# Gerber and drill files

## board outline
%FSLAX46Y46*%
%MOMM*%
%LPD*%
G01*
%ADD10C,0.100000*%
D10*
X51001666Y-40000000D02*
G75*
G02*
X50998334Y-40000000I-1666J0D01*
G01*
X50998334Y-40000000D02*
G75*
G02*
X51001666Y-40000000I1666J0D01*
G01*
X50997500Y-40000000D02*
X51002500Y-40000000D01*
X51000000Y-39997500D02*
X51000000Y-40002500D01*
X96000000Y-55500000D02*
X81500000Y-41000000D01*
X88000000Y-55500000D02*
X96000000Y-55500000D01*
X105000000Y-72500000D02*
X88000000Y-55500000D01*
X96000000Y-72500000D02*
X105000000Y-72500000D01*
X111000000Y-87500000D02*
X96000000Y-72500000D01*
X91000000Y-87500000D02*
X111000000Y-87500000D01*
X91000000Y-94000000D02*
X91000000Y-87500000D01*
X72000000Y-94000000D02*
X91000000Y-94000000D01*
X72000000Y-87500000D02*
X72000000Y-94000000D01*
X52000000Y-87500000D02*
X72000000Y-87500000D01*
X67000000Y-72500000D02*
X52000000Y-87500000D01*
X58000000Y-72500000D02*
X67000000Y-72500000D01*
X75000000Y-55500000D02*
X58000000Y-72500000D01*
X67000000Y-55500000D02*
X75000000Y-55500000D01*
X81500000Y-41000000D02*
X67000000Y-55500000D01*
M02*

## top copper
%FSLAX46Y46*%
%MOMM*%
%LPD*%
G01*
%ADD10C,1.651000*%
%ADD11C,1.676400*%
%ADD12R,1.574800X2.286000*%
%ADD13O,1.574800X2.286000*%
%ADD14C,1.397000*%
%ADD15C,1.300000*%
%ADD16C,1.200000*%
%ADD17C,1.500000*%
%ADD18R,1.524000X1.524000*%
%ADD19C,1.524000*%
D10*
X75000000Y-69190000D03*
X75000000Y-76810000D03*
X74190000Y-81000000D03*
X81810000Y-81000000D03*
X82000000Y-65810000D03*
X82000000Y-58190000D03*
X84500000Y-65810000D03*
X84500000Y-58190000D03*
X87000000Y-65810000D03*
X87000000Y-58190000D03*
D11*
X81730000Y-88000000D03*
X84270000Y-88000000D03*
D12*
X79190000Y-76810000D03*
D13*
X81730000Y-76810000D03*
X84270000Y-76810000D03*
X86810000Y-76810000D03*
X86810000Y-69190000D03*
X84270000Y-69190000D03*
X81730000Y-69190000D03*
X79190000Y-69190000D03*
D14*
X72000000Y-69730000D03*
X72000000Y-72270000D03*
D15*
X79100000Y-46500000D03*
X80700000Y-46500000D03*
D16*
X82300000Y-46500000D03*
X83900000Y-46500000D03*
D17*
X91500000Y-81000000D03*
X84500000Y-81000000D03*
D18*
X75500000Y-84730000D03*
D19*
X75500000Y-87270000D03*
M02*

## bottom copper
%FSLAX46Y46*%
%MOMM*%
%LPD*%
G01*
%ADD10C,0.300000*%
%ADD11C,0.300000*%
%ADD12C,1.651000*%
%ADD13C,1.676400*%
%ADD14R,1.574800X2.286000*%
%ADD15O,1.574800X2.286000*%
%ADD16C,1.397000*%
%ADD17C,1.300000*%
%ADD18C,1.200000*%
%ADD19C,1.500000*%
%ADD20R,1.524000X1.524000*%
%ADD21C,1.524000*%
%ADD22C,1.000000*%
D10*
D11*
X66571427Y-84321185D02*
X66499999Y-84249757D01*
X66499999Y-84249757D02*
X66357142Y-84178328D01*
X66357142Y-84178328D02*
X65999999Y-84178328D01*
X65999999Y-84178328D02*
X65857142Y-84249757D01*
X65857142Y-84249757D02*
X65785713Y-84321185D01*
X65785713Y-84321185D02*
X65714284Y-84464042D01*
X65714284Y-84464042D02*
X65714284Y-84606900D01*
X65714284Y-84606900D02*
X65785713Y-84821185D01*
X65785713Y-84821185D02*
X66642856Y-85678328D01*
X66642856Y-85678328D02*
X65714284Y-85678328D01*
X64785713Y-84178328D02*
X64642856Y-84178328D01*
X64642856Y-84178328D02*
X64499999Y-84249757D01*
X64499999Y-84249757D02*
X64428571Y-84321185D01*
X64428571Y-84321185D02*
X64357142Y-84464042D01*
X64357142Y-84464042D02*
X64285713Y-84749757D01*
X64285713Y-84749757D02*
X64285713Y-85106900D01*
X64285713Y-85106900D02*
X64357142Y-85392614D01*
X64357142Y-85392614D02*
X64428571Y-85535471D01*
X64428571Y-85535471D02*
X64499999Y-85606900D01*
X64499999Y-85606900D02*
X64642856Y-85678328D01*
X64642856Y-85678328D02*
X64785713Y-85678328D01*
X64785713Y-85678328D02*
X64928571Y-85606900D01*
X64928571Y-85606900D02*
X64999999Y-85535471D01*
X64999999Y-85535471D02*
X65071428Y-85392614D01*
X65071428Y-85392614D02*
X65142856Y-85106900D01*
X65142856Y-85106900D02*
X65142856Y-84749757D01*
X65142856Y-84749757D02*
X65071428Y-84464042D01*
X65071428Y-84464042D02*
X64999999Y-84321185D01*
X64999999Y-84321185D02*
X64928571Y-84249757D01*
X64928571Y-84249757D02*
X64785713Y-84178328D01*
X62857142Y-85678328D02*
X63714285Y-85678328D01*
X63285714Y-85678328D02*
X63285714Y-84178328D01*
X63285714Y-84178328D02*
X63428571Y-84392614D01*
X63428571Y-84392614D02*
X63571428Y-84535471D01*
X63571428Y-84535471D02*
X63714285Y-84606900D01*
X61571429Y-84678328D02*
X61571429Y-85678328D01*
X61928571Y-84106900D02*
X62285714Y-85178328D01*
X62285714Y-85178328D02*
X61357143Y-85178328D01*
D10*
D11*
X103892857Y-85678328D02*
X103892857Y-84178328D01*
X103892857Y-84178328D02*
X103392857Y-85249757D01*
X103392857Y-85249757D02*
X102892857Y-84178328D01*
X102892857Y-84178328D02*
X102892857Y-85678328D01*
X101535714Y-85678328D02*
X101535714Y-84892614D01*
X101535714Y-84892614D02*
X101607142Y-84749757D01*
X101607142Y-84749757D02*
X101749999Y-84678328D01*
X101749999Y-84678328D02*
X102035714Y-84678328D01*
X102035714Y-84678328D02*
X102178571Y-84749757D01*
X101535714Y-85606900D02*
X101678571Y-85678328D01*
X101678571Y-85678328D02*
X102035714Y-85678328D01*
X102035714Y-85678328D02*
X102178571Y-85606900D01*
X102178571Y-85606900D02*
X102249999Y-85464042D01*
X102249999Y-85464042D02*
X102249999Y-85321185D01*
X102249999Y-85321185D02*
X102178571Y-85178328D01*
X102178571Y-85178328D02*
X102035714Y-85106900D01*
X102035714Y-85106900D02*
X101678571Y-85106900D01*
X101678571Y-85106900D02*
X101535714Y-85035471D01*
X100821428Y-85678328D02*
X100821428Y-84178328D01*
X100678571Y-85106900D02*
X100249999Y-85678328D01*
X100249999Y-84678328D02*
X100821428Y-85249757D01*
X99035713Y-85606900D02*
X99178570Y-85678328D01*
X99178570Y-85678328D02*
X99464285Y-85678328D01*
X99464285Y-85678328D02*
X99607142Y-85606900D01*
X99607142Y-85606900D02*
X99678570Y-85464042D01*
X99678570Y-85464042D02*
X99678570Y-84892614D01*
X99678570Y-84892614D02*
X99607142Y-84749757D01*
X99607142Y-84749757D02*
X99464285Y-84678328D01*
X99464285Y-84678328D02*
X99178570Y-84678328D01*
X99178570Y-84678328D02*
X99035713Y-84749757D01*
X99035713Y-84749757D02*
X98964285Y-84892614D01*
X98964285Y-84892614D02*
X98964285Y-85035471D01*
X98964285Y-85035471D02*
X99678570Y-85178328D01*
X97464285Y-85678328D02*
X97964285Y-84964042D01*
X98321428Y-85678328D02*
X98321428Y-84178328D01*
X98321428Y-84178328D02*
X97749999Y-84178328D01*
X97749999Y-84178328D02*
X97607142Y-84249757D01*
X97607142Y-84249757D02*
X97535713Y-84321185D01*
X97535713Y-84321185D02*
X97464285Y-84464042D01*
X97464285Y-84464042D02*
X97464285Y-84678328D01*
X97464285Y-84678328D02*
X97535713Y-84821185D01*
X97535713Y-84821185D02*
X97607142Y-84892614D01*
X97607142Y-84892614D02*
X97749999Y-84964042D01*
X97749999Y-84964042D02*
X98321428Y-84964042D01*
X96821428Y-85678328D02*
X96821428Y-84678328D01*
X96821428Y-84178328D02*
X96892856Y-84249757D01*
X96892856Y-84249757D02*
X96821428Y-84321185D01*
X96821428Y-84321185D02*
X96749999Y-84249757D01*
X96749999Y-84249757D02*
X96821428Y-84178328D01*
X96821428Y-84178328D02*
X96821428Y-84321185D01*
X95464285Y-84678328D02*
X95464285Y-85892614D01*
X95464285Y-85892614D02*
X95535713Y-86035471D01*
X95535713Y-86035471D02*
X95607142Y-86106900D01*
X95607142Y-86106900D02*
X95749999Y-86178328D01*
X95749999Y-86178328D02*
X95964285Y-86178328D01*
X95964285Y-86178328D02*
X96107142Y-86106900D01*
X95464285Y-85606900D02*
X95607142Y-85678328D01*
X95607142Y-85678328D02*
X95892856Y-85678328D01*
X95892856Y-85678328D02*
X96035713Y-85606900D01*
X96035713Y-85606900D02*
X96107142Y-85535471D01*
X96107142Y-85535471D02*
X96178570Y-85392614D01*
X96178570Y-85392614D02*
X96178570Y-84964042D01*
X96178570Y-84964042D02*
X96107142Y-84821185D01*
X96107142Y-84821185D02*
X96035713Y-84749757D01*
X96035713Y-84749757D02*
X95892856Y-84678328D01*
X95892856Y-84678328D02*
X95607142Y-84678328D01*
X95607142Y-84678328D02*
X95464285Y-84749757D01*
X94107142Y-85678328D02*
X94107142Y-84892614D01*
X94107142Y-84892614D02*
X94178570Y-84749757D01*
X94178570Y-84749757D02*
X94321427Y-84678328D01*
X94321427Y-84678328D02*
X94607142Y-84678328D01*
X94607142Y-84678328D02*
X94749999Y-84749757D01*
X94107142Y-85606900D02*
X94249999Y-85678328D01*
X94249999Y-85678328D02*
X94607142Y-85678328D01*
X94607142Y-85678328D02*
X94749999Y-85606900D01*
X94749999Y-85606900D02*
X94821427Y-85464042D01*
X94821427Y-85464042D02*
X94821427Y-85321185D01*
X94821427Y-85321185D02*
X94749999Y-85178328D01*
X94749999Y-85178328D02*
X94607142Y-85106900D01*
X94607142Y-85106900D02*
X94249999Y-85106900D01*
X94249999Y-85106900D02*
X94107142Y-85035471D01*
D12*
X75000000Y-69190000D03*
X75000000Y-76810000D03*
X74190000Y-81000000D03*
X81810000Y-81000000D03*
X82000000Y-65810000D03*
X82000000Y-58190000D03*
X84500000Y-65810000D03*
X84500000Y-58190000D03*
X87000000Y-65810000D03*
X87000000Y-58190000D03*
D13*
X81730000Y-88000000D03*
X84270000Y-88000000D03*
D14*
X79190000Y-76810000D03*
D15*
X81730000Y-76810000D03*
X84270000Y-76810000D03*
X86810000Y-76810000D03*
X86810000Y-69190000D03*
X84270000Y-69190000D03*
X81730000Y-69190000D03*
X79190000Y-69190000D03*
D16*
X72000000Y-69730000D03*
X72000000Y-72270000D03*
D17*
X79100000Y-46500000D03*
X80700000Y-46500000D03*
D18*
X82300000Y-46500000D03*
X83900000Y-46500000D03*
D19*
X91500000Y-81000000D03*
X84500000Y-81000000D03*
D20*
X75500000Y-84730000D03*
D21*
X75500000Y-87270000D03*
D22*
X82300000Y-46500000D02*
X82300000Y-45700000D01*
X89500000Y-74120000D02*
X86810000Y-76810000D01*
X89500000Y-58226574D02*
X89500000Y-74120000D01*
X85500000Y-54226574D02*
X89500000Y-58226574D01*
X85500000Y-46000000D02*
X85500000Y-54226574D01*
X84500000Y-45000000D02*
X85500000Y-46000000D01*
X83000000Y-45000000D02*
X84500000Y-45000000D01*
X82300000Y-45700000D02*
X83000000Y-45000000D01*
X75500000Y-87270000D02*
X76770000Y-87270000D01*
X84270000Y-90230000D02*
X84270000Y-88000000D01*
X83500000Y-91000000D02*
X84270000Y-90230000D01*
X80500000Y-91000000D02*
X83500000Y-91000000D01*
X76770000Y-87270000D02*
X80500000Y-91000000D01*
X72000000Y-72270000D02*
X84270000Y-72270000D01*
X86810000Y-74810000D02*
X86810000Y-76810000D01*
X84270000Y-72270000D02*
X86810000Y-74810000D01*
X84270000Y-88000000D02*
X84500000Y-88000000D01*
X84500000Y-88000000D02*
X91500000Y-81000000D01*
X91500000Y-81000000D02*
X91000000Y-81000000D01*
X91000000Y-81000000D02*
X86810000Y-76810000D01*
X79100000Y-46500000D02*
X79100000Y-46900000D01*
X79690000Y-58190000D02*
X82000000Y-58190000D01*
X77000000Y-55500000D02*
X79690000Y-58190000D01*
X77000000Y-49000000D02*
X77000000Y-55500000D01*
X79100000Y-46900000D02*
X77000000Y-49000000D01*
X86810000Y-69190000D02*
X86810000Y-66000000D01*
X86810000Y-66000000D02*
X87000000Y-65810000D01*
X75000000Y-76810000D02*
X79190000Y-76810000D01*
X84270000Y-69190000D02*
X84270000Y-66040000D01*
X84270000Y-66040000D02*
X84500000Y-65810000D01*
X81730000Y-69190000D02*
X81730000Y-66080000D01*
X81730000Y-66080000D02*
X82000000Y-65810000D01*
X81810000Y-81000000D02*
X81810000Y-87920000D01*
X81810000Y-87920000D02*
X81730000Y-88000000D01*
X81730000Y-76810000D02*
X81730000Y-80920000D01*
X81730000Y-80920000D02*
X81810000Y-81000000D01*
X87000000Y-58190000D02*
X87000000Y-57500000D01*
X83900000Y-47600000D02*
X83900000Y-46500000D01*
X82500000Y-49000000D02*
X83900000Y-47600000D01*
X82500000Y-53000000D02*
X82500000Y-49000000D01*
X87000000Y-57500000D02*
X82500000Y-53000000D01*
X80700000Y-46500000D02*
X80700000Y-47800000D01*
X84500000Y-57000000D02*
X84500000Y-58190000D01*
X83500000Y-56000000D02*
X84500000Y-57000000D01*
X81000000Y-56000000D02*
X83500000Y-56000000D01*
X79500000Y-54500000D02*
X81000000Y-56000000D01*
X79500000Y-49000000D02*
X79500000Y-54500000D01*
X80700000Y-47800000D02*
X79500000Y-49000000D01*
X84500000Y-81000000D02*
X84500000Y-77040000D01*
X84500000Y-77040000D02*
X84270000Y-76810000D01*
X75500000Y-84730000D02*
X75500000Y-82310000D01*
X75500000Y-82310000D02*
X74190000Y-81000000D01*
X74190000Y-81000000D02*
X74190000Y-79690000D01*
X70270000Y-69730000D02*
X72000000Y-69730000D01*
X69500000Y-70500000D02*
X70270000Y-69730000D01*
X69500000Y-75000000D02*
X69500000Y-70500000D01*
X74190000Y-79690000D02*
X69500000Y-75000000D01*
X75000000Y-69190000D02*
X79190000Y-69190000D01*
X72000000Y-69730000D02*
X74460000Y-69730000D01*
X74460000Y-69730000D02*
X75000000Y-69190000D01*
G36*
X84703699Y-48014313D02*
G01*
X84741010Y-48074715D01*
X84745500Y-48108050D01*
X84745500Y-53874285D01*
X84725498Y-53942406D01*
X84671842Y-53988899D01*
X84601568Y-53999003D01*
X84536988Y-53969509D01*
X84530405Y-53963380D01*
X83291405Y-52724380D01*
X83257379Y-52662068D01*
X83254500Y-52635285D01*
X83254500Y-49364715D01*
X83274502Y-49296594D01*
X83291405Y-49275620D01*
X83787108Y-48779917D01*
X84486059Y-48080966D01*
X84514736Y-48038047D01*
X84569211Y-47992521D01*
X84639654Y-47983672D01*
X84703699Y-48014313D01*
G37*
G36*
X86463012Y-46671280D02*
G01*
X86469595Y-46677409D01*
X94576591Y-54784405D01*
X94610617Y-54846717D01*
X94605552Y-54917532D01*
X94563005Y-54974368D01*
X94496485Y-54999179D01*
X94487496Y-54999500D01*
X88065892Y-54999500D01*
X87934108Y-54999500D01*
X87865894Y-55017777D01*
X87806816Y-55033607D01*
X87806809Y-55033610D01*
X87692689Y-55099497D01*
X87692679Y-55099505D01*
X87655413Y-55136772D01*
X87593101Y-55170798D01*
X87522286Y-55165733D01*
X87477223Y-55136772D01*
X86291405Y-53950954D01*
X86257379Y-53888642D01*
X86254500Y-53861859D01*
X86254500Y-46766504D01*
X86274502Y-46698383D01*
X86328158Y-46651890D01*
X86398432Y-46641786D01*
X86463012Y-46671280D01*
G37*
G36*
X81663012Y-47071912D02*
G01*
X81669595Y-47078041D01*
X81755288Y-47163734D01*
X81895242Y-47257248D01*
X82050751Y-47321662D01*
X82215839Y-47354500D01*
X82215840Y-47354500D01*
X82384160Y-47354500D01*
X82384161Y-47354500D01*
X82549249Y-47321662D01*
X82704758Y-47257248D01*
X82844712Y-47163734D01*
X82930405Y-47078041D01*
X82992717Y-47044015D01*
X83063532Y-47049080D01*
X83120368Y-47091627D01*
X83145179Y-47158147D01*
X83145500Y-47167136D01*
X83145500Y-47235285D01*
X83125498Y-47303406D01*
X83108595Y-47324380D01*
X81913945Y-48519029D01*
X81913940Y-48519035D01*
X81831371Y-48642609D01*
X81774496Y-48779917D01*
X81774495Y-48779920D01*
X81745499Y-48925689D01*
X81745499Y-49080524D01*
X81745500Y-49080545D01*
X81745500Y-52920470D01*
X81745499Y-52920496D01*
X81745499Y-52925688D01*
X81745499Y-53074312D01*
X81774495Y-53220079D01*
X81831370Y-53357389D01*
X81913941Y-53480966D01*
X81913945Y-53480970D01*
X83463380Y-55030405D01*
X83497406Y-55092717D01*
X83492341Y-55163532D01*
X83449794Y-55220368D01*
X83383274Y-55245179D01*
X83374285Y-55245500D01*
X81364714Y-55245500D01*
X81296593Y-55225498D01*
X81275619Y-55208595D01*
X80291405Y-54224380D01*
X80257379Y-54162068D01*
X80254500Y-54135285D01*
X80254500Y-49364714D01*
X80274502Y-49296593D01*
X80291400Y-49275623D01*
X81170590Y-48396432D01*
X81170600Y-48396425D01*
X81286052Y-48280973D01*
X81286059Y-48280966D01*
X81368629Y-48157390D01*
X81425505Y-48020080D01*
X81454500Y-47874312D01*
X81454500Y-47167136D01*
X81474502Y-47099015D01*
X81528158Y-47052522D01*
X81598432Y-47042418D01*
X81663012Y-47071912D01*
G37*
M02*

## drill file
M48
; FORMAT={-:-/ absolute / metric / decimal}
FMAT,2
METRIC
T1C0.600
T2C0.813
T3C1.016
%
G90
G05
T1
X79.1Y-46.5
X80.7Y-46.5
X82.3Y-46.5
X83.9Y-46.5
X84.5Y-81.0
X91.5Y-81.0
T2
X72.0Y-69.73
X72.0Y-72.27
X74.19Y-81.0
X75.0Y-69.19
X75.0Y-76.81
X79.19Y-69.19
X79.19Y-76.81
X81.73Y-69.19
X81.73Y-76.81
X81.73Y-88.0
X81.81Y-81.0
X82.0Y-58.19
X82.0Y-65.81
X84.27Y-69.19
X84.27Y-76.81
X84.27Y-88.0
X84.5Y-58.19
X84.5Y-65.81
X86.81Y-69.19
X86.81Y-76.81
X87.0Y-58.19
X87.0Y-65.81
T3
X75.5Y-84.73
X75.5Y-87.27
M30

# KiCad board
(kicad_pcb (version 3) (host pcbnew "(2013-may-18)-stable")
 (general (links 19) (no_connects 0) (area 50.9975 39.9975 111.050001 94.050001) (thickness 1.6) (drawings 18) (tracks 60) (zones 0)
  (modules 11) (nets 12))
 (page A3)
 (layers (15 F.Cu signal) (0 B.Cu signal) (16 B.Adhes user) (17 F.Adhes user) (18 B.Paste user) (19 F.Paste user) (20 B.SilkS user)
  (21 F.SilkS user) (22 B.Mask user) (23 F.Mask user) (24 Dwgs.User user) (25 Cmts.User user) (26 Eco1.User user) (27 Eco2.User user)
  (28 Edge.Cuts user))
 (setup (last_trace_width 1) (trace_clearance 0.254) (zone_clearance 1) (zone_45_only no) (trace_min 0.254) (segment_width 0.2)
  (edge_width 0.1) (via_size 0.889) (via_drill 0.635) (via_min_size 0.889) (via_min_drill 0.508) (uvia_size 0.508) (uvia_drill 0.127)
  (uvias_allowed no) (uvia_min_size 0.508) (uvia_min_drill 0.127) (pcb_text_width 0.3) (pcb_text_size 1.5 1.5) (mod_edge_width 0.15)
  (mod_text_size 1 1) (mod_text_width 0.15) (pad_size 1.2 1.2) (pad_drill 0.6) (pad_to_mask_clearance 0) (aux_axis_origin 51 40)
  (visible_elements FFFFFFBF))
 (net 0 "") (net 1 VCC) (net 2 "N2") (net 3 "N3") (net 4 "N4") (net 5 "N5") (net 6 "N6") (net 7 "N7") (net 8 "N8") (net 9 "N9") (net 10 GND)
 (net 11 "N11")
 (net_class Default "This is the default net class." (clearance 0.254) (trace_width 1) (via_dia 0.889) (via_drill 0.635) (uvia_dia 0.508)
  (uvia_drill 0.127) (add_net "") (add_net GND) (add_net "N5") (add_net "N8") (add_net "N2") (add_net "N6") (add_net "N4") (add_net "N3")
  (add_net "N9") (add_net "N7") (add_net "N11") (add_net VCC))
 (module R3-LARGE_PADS (layer F.Cu) (at 75 73 270) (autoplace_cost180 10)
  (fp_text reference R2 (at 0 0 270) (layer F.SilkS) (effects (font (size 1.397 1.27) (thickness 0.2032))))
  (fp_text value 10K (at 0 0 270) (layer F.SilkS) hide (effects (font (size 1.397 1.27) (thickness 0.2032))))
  (pad 1 thru_hole circle (at -3.81 0 270) (size 1.651 1.651) (drill 0.8128) (layers *.Cu *.Mask F.SilkS) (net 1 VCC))
  (pad 2 thru_hole circle (at 3.81 0 270) (size 1.651 1.651) (drill 0.8128) (layers *.Cu *.Mask F.SilkS) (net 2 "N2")))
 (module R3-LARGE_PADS (layer F.Cu) (at 78 81) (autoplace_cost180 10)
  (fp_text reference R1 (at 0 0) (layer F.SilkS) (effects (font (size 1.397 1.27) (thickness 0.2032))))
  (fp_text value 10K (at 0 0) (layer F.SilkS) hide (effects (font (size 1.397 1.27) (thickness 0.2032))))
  (pad 1 thru_hole circle (at -3.81 0) (size 1.651 1.651) (drill 0.8128) (layers *.Cu *.Mask F.SilkS) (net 1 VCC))
  (pad 2 thru_hole circle (at 3.81 0) (size 1.651 1.651) (drill 0.8128) (layers *.Cu *.Mask F.SilkS) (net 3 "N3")))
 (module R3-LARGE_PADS (layer F.Cu) (at 82 62 90) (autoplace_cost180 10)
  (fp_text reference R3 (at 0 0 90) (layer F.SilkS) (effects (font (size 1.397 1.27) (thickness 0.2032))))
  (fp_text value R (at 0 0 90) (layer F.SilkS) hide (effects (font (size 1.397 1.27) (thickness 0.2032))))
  (pad 1 thru_hole circle (at -3.81 0 90) (size 1.651 1.651) (drill 0.8128) (layers *.Cu *.Mask F.SilkS) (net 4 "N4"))
  (pad 2 thru_hole circle (at 3.81 0 90) (size 1.651 1.651) (drill 0.8128) (layers *.Cu *.Mask F.SilkS) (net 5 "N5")))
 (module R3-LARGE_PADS (layer F.Cu) (at 84.5 62 90) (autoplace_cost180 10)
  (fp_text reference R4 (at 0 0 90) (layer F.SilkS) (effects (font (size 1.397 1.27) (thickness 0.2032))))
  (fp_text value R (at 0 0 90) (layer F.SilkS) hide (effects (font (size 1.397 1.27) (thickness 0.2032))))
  (pad 1 thru_hole circle (at -3.81 0 90) (size 1.651 1.651) (drill 0.8128) (layers *.Cu *.Mask F.SilkS) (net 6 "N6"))
  (pad 2 thru_hole circle (at 3.81 0 90) (size 1.651 1.651) (drill 0.8128) (layers *.Cu *.Mask F.SilkS) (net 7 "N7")))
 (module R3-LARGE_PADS (layer F.Cu) (at 87 62 90) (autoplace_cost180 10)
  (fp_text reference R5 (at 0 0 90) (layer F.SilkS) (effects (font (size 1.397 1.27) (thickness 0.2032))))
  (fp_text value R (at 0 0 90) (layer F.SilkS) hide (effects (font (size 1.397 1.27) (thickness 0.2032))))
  (pad 1 thru_hole circle (at -3.81 0 90) (size 1.651 1.651) (drill 0.8128) (layers *.Cu *.Mask F.SilkS) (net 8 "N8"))
  (pad 2 thru_hole circle (at 3.81 0 90) (size 1.651 1.651) (drill 0.8128) (layers *.Cu *.Mask F.SilkS) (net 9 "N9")))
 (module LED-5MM (layer F.Cu) (at 83 88)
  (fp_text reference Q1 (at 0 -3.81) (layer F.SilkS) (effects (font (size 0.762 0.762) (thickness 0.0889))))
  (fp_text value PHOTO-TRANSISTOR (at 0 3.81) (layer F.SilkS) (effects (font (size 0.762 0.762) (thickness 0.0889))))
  (pad 1 thru_hole circle (at -1.27 0) (size 1.6764 1.6764) (drill 0.8128) (layers *.Cu *.Mask F.SilkS) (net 3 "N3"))
  (pad 2 thru_hole circle (at 1.27 0) (size 1.6764 1.6764) (drill 0.8128) (layers *.Cu *.Mask F.SilkS) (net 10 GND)))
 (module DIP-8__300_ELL (layer F.Cu) (at 83 73)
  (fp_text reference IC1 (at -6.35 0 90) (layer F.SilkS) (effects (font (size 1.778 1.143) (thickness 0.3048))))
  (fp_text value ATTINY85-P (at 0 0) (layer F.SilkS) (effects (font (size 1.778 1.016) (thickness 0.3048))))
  (pad 1 thru_hole rect (at -3.81 3.81) (size 1.5748 2.286) (drill 0.8128) (layers *.Cu *.Mask F.SilkS) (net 2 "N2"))
  (pad 2 thru_hole oval (at -1.27 3.81) (size 1.5748 2.286) (drill 0.8128) (layers *.Cu *.Mask F.SilkS) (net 3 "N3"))
  (pad 3 thru_hole oval (at 1.27 3.81) (size 1.5748 2.286) (drill 0.8128) (layers *.Cu *.Mask F.SilkS) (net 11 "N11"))
  (pad 4 thru_hole oval (at 3.81 3.81) (size 1.5748 2.286) (drill 0.8128) (layers *.Cu *.Mask F.SilkS) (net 10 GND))
  (pad 5 thru_hole oval (at 3.81 -3.81) (size 1.5748 2.286) (drill 0.8128) (layers *.Cu *.Mask F.SilkS) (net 8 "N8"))
  (pad 6 thru_hole oval (at 1.27 -3.81) (size 1.5748 2.286) (drill 0.8128) (layers *.Cu *.Mask F.SilkS) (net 6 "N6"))
  (pad 7 thru_hole oval (at -1.27 -3.81) (size 1.5748 2.286) (drill 0.8128) (layers *.Cu *.Mask F.SilkS) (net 4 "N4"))
  (pad 8 thru_hole oval (at -3.81 -3.81) (size 1.5748 2.286) (drill 0.8128) (layers *.Cu *.Mask F.SilkS) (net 1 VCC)))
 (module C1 (layer F.Cu) (at 72 71 270)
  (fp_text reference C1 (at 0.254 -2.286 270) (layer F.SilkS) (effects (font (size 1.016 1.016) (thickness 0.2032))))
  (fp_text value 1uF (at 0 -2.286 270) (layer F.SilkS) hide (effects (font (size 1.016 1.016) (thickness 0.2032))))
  (pad 1 thru_hole circle (at -1.27 0 270) (size 1.397 1.397) (drill 0.8128) (layers *.Cu *.Mask F.SilkS) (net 1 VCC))
  (pad 2 thru_hole circle (at 1.27 0 270) (size 1.397 1.397) (drill 0.8128) (layers *.Cu *.Mask F.SilkS) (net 10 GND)))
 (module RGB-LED (layer F.Cu) (at 81.5 46.5)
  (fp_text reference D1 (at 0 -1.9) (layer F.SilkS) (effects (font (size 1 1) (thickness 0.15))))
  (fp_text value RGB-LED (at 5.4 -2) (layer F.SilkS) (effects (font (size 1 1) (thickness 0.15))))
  (pad 1 thru_hole circle (at -2.4 0) (size 1.3 1.3) (drill 0.6) (layers *.Cu *.Mask F.SilkS) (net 5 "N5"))
  (pad 2 thru_hole circle (at -0.8 0) (size 1.3 1.3) (drill 0.6) (layers *.Cu *.Mask F.SilkS) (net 7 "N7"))
  (pad 3 thru_hole circle (at 0.8 0) (size 1.2 1.2) (drill 0.6) (layers *.Cu *.Mask F.SilkS) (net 10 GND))
  (pad 4 thru_hole circle (at 2.4 0) (size 1.2 1.2) (drill 0.6) (layers *.Cu *.Mask F.SilkS) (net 9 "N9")))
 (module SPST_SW (layer F.Cu) (at 88 81 180)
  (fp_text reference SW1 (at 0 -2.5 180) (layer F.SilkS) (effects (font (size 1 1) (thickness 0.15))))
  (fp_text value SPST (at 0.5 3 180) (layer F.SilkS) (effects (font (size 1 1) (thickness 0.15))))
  (pad 1 thru_hole circle (at -3.5 0 180) (size 1.5 1.5) (drill 0.6) (layers *.Cu *.Mask F.SilkS) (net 10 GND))
  (pad 2 thru_hole circle (at 3.5 0 180) (size 1.5 1.5) (drill 0.6) (layers *.Cu *.Mask F.SilkS) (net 11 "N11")))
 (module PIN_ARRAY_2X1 (layer F.Cu) (at 75.5 86 270)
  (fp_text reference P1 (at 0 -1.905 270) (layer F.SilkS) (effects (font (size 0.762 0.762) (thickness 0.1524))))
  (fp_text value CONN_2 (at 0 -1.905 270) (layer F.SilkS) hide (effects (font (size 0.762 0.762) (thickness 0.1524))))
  (pad 1 thru_hole rect (at -1.27 0 270) (size 1.524 1.524) (drill 1.016) (layers *.Cu *.Mask F.SilkS) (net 1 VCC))
  (pad 2 thru_hole circle (at 1.27 0 270) (size 1.524 1.524) (drill 1.016) (layers *.Cu *.Mask F.SilkS) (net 10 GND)))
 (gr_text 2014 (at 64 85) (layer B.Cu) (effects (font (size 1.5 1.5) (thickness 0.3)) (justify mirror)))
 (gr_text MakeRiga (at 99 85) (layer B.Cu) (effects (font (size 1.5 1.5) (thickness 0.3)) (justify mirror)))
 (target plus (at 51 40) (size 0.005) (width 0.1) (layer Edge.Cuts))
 (gr_line (start 96 55.5) (end 81.5 41) (angle 90) (layer Edge.Cuts) (width 0.1))
 (gr_line (start 88 55.5) (end 96 55.5) (angle 90) (layer Edge.Cuts) (width 0.1))
 (gr_line (start 105 72.5) (end 88 55.5) (angle 90) (layer Edge.Cuts) (width 0.1))
 (gr_line (start 96 72.5) (end 105 72.5) (angle 90) (layer Edge.Cuts) (width 0.1))
 (gr_line (start 111 87.5) (end 96 72.5) (angle 90) (layer Edge.Cuts) (width 0.1))
 (gr_line (start 91 87.5) (end 111 87.5) (angle 90) (layer Edge.Cuts) (width 0.1))
 (gr_line (start 91 94) (end 91 87.5) (angle 90) (layer Edge.Cuts) (width 0.1))
 (gr_line (start 72 94) (end 91 94) (angle 90) (layer Edge.Cuts) (width 0.1))
 (gr_line (start 72 87.5) (end 72 94) (angle 90) (layer Edge.Cuts) (width 0.1))
 (gr_line (start 52 87.5) (end 72 87.5) (angle 90) (layer Edge.Cuts) (width 0.1))
 (gr_line (start 67 72.5) (end 52 87.5) (angle 90) (layer Edge.Cuts) (width 0.1))
 (gr_line (start 58 72.5) (end 67 72.5) (angle 90) (layer Edge.Cuts) (width 0.1))
 (gr_line (start 75 55.5) (end 58 72.5) (angle 90) (layer Edge.Cuts) (width 0.1))
 (gr_line (start 67 55.5) (end 75 55.5) (angle 90) (layer Edge.Cuts) (width 0.1))
 (gr_line (start 81.5 41) (end 67 55.5) (angle 90) (layer Edge.Cuts) (width 0.1))
 (segment (start 82.3 46.5) (end 82.3 45.7) (width 1) (layer B.Cu) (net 10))
 (segment (start 89.5 74.12) (end 86.81 76.81) (width 1) (layer B.Cu) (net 10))
 (segment (start 89.5 58.226574) (end 89.5 74.12) (width 1) (layer B.Cu) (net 10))
 (segment (start 85.5 54.226574) (end 89.5 58.226574) (width 1) (layer B.Cu) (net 10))
 (segment (start 85.5 46) (end 85.5 54.226574) (width 1) (layer B.Cu) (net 10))
 (segment (start 84.5 45) (end 85.5 46) (width 1) (layer B.Cu) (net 10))
 (segment (start 83 45) (end 84.5 45) (width 1) (layer B.Cu) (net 10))
 (segment (start 82.3 45.7) (end 83 45) (width 1) (layer B.Cu) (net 10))
 (segment (start 75.5 87.27) (end 76.77 87.27) (width 1) (layer B.Cu) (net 10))
 (segment (start 84.27 90.23) (end 84.27 88) (width 1) (layer B.Cu) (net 10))
 (segment (start 83.5 91) (end 84.27 90.23) (width 1) (layer B.Cu) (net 10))
 (segment (start 80.5 91) (end 83.5 91) (width 1) (layer B.Cu) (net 10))
 (segment (start 76.77 87.27) (end 80.5 91) (width 1) (layer B.Cu) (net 10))
 (segment (start 72 72.27) (end 84.27 72.27) (width 1) (layer B.Cu) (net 10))
 (segment (start 86.81 74.81) (end 86.81 76.81) (width 1) (layer B.Cu) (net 10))
 (segment (start 84.27 72.27) (end 86.81 74.81) (width 1) (layer B.Cu) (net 10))
 (segment (start 84.27 88) (end 84.5 88) (width 1) (layer B.Cu) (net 10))
 (segment (start 84.5 88) (end 91.5 81) (width 1) (layer B.Cu) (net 10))
 (segment (start 91.5 81) (end 91 81) (width 1) (layer B.Cu) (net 10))
 (segment (start 91 81) (end 86.81 76.81) (width 1) (layer B.Cu) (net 10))
 (segment (start 79.1 46.5) (end 79.1 46.9) (width 1) (layer B.Cu) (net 5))
 (segment (start 79.69 58.19) (end 82 58.19) (width 1) (layer B.Cu) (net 5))
 (segment (start 77 55.5) (end 79.69 58.19) (width 1) (layer B.Cu) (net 5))
 (segment (start 77 49) (end 77 55.5) (width 1) (layer B.Cu) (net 5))
 (segment (start 79.1 46.9) (end 77 49) (width 1) (layer B.Cu) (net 5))
 (segment (start 86.81 69.19) (end 86.81 66) (width 1) (layer B.Cu) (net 8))
 (segment (start 86.81 66) (end 87 65.81) (width 1) (layer B.Cu) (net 8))
 (segment (start 75 76.81) (end 79.19 76.81) (width 1) (layer B.Cu) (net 2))
 (segment (start 84.27 69.19) (end 84.27 66.04) (width 1) (layer B.Cu) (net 6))
 (segment (start 84.27 66.04) (end 84.5 65.81) (width 1) (layer B.Cu) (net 6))
 (segment (start 81.73 69.19) (end 81.73 66.08) (width 1) (layer B.Cu) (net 4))
 (segment (start 81.73 66.08) (end 82 65.81) (width 1) (layer B.Cu) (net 4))
 (segment (start 81.81 81) (end 81.81 87.92) (width 1) (layer B.Cu) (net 3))
 (segment (start 81.81 87.92) (end 81.73 88) (width 1) (layer B.Cu) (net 3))
 (segment (start 81.73 76.81) (end 81.73 80.92) (width 1) (layer B.Cu) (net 3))
 (segment (start 81.73 80.92) (end 81.81 81) (width 1) (layer B.Cu) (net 3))
 (segment (start 87 58.19) (end 87 57.5) (width 1) (layer B.Cu) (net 9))
 (segment (start 83.9 47.6) (end 83.9 46.5) (width 1) (layer B.Cu) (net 9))
 (segment (start 82.5 49) (end 83.9 47.6) (width 1) (layer B.Cu) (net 9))
 (segment (start 82.5 53) (end 82.5 49) (width 1) (layer B.Cu) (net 9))
 (segment (start 87 57.5) (end 82.5 53) (width 1) (layer B.Cu) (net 9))
 (segment (start 80.7 46.5) (end 80.7 47.8) (width 1) (layer B.Cu) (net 7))
 (segment (start 84.5 57) (end 84.5 58.19) (width 1) (layer B.Cu) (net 7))
 (segment (start 83.5 56) (end 84.5 57) (width 1) (layer B.Cu) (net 7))
 (segment (start 81 56) (end 83.5 56) (width 1) (layer B.Cu) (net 7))
 (segment (start 79.5 54.5) (end 81 56) (width 1) (layer B.Cu) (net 7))
 (segment (start 79.5 49) (end 79.5 54.5) (width 1) (layer B.Cu) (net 7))
 (segment (start 80.7 47.8) (end 79.5 49) (width 1) (layer B.Cu) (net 7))
 (segment (start 84.5 81) (end 84.5 77.04) (width 1) (layer B.Cu) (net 11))
 (segment (start 84.5 77.04) (end 84.27 76.81) (width 1) (layer B.Cu) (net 11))
 (segment (start 75.5 84.73) (end 75.5 82.31) (width 1) (layer B.Cu) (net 1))
 (segment (start 75.5 82.31) (end 74.19 81) (width 1) (layer B.Cu) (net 1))
 (segment (start 74.19 81) (end 74.19 79.69) (width 1) (layer B.Cu) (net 1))
 (segment (start 70.27 69.73) (end 72 69.73) (width 1) (layer B.Cu) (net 1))
 (segment (start 69.5 70.5) (end 70.27 69.73) (width 1) (layer B.Cu) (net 1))
 (segment (start 69.5 75) (end 69.5 70.5) (width 1) (layer B.Cu) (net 1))
 (segment (start 74.19 79.69) (end 69.5 75) (width 1) (layer B.Cu) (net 1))
 (segment (start 75 69.19) (end 79.19 69.19) (width 1) (layer B.Cu) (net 1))
 (segment (start 72 69.73) (end 74.46 69.73) (width 1) (layer B.Cu) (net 1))
 (segment (start 74.46 69.73) (end 75 69.19) (width 1) (layer B.Cu) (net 1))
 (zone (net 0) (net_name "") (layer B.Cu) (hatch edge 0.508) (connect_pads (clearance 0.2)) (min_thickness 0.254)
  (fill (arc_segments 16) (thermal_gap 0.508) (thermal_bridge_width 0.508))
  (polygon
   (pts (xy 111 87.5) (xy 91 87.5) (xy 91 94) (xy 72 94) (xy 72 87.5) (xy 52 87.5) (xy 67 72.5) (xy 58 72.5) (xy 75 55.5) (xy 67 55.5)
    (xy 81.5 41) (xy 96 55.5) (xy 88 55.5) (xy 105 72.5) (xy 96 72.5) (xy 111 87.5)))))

